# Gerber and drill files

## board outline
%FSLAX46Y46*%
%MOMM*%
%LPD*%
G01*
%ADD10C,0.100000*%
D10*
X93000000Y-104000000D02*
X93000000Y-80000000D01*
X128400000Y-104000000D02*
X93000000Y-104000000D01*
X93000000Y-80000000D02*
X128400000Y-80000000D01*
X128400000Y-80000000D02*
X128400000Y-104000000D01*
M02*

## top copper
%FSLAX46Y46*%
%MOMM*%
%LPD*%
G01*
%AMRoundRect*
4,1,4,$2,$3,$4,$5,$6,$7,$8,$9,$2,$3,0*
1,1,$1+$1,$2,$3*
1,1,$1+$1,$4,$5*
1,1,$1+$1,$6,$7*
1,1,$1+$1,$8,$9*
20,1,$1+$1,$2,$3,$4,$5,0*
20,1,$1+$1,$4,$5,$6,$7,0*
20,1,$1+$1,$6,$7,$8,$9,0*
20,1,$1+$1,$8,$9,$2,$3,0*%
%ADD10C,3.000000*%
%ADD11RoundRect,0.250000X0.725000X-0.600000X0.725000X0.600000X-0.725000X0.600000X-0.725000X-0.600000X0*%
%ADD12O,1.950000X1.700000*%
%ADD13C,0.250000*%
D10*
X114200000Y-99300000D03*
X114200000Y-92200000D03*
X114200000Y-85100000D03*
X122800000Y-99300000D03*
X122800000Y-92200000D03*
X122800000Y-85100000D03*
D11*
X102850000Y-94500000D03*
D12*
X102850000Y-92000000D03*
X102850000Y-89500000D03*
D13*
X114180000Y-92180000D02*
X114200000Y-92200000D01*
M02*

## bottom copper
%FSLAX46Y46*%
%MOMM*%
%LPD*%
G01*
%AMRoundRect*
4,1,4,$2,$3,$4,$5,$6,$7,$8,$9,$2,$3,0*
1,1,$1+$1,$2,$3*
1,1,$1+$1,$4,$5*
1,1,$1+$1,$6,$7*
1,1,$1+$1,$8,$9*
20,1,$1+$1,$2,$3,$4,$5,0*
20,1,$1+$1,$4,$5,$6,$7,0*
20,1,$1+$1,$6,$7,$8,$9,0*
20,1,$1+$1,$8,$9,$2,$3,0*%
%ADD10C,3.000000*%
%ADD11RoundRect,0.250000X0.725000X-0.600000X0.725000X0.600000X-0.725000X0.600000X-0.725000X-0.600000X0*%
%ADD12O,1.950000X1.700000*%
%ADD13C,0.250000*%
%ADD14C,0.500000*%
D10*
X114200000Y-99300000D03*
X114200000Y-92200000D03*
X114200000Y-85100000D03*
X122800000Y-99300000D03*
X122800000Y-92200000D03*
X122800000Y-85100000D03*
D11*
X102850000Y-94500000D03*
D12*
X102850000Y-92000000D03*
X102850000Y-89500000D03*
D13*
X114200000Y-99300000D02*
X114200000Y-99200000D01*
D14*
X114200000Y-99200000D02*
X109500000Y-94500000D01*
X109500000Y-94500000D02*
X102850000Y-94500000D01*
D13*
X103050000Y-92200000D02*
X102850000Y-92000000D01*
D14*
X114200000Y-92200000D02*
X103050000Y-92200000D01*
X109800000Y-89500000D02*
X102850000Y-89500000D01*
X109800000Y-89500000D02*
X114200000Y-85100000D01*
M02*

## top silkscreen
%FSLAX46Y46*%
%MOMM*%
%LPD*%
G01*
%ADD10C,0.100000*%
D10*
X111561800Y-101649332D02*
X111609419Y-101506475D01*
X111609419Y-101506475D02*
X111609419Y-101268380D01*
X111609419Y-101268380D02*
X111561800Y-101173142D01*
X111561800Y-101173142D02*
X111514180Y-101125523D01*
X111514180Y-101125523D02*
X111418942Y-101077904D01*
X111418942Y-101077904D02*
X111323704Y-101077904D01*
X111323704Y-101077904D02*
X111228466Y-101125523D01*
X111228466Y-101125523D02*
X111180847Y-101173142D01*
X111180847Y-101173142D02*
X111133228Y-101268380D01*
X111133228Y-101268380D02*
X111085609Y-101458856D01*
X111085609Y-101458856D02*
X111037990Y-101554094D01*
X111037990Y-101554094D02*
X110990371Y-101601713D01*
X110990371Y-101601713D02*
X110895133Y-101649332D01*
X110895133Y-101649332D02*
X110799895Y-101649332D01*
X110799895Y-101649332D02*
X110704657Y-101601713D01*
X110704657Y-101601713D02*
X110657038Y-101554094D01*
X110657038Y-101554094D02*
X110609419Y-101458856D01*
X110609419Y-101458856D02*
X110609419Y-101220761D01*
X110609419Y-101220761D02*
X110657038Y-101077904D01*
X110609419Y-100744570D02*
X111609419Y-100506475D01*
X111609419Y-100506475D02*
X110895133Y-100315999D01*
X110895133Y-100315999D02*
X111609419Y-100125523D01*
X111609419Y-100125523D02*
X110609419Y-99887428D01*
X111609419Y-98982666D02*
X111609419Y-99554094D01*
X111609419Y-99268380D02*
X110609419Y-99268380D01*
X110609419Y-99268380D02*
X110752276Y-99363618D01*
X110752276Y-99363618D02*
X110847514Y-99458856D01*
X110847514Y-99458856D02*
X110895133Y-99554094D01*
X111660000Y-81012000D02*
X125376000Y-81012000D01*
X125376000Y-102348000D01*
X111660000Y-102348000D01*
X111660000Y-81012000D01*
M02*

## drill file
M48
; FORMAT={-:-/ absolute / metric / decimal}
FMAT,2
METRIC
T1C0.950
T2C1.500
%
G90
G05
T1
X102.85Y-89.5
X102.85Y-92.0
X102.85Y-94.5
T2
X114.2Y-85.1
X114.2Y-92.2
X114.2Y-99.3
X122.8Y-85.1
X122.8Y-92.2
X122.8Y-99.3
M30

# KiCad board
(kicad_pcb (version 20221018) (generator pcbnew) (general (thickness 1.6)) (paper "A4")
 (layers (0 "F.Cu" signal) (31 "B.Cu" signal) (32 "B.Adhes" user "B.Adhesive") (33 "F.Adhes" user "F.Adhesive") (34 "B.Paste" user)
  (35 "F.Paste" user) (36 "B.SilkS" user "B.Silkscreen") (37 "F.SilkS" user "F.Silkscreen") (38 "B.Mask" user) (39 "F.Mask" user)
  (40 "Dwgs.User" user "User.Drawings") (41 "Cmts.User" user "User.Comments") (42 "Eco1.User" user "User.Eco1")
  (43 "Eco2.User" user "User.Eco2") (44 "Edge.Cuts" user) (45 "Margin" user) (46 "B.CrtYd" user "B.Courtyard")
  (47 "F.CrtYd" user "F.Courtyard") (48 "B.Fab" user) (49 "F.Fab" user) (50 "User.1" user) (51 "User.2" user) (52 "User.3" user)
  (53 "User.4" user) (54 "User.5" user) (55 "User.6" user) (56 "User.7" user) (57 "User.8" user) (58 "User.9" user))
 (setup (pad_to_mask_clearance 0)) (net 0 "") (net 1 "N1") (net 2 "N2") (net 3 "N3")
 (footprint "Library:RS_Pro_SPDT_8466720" (layer "F.Cu") (at 114.2 99.3 90)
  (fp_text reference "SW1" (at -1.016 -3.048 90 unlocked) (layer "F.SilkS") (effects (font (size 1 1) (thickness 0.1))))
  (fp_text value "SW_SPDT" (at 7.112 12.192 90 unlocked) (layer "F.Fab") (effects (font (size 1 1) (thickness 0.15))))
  (fp_rect (start -3.048 -2.54) (end 18.288 11.176) (stroke (width 0.1) (type default)) (fill none) (layer "F.SilkS"))
  (pad "1" thru_hole circle (at 0 0 90) (size 3 3) (drill 1.5) (layers "*.Cu" "*.Mask") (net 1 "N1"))
  (pad "2" thru_hole circle (at 7.1 0 90) (size 3 3) (drill 1.5) (layers "*.Cu" "*.Mask") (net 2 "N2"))
  (pad "3" thru_hole circle (at 14.2 0 90) (size 3 3) (drill 1.5) (layers "*.Cu" "*.Mask") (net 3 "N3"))
  (pad "4" thru_hole circle (at 0 8.6 90) (size 3 3) (drill 1.5) (layers "*.Cu" "*.Mask"))
  (pad "5" thru_hole circle (at 7.1 8.6 90) (size 3 3) (drill 1.5) (layers "*.Cu" "*.Mask"))
  (pad "6" thru_hole circle (at 14.2 8.6 90) (size 3 3) (drill 1.5) (layers "*.Cu" "*.Mask")))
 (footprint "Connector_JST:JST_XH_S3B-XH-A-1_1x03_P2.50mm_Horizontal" (layer "B.Cu") (at 102.85 94.5 90)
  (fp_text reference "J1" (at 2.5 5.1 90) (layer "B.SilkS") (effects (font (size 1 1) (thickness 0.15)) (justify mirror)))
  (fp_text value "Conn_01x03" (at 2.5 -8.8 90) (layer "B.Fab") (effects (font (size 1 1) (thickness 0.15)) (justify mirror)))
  (pad "1" thru_hole roundrect (at 0 0 90) (size 1.7 1.95) (drill 0.95) (layers "*.Cu" "*.Mask") (roundrect_rratio 0.147059) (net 1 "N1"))
  (pad "2" thru_hole oval (at 2.5 0 90) (size 1.7 1.95) (drill 0.95) (layers "*.Cu" "*.Mask") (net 2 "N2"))
  (pad "3" thru_hole oval (at 5 0 90) (size 1.7 1.95) (drill 0.95) (layers "*.Cu" "*.Mask") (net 3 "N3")))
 (gr_line (start 93 104) (end 93 80) (stroke (width 0.1) (type default)) (layer "Edge.Cuts"))
 (gr_line (start 128.4 104) (end 93 104) (stroke (width 0.1) (type default)) (layer "Edge.Cuts"))
 (gr_line (start 93 80) (end 128.4 80) (stroke (width 0.1) (type default)) (layer "Edge.Cuts"))
 (gr_line (start 128.4 80) (end 128.4 104) (stroke (width 0.1) (type default)) (layer "Edge.Cuts"))
 (segment (start 114.2 99.3) (end 114.2 99.2) (width 0.25) (layer "B.Cu") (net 1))
 (segment (start 114.2 99.2) (end 109.5 94.5) (width 0.5) (layer "B.Cu") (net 1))
 (segment (start 109.5 94.5) (end 102.85 94.5) (width 0.5) (layer "B.Cu") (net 1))
 (segment (start 114.18 92.18) (end 114.2 92.2) (width 0.25) (layer "F.Cu") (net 2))
 (segment (start 103.05 92.2) (end 102.85 92) (width 0.25) (layer "B.Cu") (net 2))
 (segment (start 114.2 92.2) (end 103.05 92.2) (width 0.5) (layer "B.Cu") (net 2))
 (segment (start 109.8 89.5) (end 102.85 89.5) (width 0.5) (layer "B.Cu") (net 3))
 (segment (start 109.8 89.5) (end 114.2 85.1) (width 0.5) (layer "B.Cu") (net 3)))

